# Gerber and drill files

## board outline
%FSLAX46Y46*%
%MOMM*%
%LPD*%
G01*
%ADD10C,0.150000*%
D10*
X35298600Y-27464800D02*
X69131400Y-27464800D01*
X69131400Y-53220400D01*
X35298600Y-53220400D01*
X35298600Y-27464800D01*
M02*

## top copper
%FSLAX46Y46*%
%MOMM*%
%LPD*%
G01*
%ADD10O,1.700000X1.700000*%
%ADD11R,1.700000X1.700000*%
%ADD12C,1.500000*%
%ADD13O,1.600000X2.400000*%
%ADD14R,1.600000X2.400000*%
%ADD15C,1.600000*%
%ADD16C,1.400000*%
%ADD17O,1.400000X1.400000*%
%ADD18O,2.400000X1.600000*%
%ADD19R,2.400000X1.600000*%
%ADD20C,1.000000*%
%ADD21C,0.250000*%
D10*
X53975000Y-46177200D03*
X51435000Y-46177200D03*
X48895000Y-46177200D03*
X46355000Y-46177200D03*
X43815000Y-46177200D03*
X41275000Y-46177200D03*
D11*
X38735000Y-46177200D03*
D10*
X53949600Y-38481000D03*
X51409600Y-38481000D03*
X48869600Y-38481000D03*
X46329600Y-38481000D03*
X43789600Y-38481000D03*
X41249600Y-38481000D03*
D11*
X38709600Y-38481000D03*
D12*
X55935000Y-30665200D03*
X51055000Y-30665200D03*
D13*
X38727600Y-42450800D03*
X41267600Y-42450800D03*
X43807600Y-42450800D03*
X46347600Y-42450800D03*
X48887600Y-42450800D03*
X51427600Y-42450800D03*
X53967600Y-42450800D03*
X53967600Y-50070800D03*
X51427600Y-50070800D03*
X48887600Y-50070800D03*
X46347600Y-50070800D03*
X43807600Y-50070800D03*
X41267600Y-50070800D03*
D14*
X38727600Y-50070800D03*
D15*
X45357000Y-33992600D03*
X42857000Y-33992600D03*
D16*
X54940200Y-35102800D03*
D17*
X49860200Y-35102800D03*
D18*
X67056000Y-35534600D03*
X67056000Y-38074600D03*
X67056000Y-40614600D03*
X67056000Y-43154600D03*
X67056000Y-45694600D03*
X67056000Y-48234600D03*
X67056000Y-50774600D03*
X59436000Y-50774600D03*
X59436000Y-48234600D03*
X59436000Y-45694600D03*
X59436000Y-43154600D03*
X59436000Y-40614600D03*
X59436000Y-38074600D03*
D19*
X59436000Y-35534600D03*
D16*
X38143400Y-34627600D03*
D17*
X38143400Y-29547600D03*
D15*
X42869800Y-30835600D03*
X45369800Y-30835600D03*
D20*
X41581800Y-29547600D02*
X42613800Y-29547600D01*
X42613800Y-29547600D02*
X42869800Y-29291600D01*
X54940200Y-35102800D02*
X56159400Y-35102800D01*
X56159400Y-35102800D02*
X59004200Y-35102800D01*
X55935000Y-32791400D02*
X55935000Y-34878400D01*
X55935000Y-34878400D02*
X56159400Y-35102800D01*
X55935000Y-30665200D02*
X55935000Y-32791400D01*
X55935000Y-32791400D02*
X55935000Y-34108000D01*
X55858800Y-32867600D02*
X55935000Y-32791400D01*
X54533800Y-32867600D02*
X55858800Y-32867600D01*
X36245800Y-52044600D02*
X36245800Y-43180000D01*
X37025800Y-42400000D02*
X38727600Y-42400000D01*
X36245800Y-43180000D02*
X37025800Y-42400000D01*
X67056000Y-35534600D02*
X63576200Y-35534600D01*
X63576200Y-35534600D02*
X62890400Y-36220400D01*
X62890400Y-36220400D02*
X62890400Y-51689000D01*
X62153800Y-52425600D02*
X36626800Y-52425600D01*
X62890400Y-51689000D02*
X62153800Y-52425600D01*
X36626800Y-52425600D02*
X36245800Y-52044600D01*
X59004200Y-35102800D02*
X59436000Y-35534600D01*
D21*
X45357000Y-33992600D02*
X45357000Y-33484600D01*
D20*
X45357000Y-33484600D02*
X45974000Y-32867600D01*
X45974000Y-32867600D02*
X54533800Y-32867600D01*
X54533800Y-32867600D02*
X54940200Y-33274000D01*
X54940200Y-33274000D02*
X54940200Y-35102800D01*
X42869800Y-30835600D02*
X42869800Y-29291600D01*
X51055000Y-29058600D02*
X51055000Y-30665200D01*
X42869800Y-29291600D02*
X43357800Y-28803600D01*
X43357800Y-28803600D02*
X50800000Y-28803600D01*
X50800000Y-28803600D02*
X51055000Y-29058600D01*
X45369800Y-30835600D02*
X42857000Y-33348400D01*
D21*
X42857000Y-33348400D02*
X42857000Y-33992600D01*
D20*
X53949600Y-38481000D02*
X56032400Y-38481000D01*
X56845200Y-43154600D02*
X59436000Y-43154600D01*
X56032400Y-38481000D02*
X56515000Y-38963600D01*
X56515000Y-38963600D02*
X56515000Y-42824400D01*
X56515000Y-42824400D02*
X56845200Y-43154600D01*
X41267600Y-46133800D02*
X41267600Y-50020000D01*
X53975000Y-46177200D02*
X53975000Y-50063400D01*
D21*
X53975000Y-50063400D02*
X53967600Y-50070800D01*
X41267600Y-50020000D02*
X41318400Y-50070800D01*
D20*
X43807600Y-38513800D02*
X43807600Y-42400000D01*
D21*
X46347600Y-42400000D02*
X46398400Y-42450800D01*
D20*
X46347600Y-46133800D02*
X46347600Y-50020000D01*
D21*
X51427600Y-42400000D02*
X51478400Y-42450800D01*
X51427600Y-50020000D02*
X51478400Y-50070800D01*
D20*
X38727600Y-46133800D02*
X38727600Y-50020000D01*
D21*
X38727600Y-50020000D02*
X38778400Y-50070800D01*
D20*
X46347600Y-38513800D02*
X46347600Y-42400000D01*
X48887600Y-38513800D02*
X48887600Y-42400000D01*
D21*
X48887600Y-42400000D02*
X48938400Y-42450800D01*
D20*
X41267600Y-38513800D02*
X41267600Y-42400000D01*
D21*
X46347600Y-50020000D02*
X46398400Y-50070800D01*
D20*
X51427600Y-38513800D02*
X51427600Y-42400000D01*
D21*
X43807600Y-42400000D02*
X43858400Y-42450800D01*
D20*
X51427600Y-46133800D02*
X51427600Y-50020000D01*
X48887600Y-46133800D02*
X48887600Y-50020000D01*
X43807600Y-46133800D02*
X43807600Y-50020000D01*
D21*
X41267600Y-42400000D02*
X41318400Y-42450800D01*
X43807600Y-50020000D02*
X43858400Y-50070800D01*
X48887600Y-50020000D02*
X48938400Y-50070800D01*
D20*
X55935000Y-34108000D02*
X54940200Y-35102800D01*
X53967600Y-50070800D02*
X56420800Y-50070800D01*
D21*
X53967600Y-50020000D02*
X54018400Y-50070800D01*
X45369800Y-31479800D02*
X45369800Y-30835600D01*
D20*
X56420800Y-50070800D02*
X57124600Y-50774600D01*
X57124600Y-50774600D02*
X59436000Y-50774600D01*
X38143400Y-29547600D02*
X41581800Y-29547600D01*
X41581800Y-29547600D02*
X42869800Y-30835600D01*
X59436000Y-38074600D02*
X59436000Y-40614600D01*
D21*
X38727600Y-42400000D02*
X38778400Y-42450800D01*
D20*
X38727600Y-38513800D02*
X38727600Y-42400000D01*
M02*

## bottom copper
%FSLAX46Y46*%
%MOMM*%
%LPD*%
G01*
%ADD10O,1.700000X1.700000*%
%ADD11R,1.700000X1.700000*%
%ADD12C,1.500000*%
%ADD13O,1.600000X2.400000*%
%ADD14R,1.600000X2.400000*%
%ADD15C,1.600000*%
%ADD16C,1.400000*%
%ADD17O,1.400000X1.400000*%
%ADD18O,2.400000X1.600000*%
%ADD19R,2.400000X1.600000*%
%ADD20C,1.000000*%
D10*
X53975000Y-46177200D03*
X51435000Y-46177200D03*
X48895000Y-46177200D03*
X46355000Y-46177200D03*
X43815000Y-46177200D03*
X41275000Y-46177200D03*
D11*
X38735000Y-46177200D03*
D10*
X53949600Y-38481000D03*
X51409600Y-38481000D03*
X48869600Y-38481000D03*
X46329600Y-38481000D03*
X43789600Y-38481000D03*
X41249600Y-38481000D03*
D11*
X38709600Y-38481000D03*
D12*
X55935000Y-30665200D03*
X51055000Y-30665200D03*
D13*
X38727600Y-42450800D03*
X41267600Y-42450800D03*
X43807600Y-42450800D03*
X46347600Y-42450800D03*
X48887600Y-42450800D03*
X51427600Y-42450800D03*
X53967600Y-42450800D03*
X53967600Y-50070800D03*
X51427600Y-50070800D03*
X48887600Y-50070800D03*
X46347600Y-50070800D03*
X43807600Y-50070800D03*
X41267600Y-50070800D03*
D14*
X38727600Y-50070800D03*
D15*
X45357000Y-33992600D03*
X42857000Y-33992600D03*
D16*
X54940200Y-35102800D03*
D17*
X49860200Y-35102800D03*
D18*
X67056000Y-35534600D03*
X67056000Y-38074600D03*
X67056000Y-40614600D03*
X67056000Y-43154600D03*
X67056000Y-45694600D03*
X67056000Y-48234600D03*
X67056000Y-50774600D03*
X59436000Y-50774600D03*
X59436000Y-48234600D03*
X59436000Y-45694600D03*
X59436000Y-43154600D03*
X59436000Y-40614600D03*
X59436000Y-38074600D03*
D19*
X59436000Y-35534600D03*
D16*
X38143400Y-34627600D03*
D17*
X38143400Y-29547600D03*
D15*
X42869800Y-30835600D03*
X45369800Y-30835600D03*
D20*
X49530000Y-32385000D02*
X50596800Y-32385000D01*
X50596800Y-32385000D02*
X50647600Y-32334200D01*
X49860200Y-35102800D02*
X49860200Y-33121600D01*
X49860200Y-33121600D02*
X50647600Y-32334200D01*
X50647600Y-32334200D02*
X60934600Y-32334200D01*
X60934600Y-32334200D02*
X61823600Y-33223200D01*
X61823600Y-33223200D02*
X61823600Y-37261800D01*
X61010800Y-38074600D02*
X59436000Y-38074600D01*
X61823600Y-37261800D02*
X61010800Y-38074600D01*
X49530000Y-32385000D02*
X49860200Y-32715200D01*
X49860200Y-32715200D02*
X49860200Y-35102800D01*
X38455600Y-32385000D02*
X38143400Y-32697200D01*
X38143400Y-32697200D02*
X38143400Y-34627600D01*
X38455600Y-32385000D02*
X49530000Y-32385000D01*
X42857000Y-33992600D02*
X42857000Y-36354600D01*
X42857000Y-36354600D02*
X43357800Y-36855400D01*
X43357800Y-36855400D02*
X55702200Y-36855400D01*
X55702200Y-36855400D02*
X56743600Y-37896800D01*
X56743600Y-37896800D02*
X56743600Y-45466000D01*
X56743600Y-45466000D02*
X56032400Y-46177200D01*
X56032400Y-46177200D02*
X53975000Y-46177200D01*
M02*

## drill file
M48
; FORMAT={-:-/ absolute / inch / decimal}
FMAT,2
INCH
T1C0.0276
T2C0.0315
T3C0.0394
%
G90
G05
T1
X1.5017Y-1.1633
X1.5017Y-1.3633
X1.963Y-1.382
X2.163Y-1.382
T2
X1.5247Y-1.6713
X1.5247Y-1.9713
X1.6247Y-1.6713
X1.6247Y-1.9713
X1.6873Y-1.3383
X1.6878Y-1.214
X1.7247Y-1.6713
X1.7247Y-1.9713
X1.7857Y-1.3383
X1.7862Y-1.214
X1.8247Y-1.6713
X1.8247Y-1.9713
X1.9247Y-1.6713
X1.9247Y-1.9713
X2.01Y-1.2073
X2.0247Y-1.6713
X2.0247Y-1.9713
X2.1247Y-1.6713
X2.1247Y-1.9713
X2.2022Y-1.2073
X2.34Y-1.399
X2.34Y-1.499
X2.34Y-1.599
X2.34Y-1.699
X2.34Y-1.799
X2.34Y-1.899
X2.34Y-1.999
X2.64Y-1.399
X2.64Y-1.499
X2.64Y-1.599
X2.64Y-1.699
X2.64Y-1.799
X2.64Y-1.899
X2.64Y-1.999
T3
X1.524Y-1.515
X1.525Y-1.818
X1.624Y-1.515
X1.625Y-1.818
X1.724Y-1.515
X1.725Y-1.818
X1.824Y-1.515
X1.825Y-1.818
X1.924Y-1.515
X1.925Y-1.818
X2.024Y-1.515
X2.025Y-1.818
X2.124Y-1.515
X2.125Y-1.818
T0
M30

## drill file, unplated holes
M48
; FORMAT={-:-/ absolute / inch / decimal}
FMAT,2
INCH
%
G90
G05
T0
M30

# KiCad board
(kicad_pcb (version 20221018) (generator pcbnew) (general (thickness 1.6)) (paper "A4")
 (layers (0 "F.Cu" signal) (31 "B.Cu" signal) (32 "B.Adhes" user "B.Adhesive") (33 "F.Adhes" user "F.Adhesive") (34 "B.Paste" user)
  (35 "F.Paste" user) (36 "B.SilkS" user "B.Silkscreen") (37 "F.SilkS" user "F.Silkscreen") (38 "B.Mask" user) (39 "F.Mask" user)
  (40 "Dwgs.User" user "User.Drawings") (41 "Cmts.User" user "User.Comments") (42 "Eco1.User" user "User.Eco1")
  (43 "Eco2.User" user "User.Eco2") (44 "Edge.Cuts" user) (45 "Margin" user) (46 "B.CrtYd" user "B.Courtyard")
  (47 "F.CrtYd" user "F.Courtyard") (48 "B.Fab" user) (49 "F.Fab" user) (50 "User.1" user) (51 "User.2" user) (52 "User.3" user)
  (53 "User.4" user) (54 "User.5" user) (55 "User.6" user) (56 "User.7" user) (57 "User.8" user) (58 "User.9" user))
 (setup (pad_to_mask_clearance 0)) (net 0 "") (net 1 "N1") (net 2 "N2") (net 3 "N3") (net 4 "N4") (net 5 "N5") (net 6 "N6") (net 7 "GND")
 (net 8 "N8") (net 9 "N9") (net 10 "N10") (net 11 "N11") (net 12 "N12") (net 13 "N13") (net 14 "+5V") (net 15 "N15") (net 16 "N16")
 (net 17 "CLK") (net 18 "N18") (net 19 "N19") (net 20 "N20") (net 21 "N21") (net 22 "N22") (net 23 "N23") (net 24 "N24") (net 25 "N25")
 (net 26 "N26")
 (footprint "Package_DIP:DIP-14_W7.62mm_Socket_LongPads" (layer "F.Cu") (at 38.7276 50.0708 90)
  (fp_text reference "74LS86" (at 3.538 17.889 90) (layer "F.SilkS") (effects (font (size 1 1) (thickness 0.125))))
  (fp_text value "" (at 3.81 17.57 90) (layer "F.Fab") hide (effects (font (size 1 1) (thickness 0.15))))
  (pad "1" thru_hole rect (at 0 0 90) (size 2.4 1.6) (drill 0.8) (layers "*.Cu" "*.Mask") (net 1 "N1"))
  (pad "2" thru_hole oval (at 0 2.54 90) (size 2.4 1.6) (drill 0.8) (layers "*.Cu" "*.Mask") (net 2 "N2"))
  (pad "3" thru_hole oval (at 0 5.08 90) (size 2.4 1.6) (drill 0.8) (layers "*.Cu" "*.Mask") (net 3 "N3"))
  (pad "4" thru_hole oval (at 0 7.62 90) (size 2.4 1.6) (drill 0.8) (layers "*.Cu" "*.Mask") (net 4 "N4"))
  (pad "5" thru_hole oval (at 0 10.16 90) (size 2.4 1.6) (drill 0.8) (layers "*.Cu" "*.Mask") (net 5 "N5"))
  (pad "6" thru_hole oval (at 0 12.7 90) (size 2.4 1.6) (drill 0.8) (layers "*.Cu" "*.Mask") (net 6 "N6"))
  (pad "7" thru_hole oval (at 0 15.24 90) (size 2.4 1.6) (drill 0.8) (layers "*.Cu" "*.Mask") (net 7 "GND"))
  (pad "8" thru_hole oval (at 7.62 15.24 90) (size 2.4 1.6) (drill 0.8) (layers "*.Cu" "*.Mask") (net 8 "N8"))
  (pad "9" thru_hole oval (at 7.62 12.7 90) (size 2.4 1.6) (drill 0.8) (layers "*.Cu" "*.Mask") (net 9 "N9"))
  (pad "10" thru_hole oval (at 7.62 10.16 90) (size 2.4 1.6) (drill 0.8) (layers "*.Cu" "*.Mask") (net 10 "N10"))
  (pad "11" thru_hole oval (at 7.62 7.62 90) (size 2.4 1.6) (drill 0.8) (layers "*.Cu" "*.Mask") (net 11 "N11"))
  (pad "12" thru_hole oval (at 7.62 5.08 90) (size 2.4 1.6) (drill 0.8) (layers "*.Cu" "*.Mask") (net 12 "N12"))
  (pad "13" thru_hole oval (at 7.62 2.54 90) (size 2.4 1.6) (drill 0.8) (layers "*.Cu" "*.Mask") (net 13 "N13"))
  (pad "14" thru_hole oval (at 7.62 0 90) (size 2.4 1.6) (drill 0.8) (layers "*.Cu" "*.Mask") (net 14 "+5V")))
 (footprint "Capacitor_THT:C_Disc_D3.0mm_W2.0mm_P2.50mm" (layer "F.Cu") (at 45.357 33.9926 180)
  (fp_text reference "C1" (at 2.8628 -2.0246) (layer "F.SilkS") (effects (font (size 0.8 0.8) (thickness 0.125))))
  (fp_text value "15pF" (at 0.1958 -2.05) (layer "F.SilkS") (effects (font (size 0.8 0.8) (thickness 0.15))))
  (pad "1" thru_hole circle (at 0 0 180) (size 1.6 1.6) (drill 0.8) (layers "*.Cu" "*.Mask") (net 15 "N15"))
  (pad "2" thru_hole circle (at 2.5 0 180) (size 1.6 1.6) (drill 0.8) (layers "*.Cu" "*.Mask") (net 7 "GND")))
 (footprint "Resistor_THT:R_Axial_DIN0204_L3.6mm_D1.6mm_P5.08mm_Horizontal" (layer "F.Cu") (at 54.9402 35.1028 180)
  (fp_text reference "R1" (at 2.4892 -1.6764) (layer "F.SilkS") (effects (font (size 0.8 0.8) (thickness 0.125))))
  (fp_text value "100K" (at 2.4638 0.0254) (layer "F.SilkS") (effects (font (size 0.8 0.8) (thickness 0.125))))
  (pad "1" thru_hole circle (at 0 0 180) (size 1.4 1.4) (drill 0.7) (layers "*.Cu" "*.Mask") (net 15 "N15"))
  (pad "2" thru_hole oval (at 5.08 0 180) (size 1.4 1.4) (drill 0.7) (layers "*.Cu" "*.Mask") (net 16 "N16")))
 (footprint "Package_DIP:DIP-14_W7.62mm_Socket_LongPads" (layer "F.Cu") (at 59.436 35.5346)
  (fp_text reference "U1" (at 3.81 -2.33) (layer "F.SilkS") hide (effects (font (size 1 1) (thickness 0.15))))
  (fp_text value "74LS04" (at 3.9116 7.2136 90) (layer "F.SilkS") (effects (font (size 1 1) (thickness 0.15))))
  (pad "1" thru_hole rect (at 0 0) (size 2.4 1.6) (drill 0.8) (layers "*.Cu" "*.Mask") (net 15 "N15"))
  (pad "2" thru_hole oval (at 0 2.54) (size 2.4 1.6) (drill 0.8) (layers "*.Cu" "*.Mask") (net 16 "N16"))
  (pad "3" thru_hole oval (at 0 5.08) (size 2.4 1.6) (drill 0.8) (layers "*.Cu" "*.Mask") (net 16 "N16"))
  (pad "4" thru_hole oval (at 0 7.62) (size 2.4 1.6) (drill 0.8) (layers "*.Cu" "*.Mask") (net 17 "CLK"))
  (pad "5" thru_hole oval (at 0 10.16) (size 2.4 1.6) (drill 0.8) (layers "*.Cu" "*.Mask") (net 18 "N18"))
  (pad "6" thru_hole oval (at 0 12.7) (size 2.4 1.6) (drill 0.8) (layers "*.Cu" "*.Mask") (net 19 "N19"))
  (pad "7" thru_hole oval (at 0 15.24) (size 2.4 1.6) (drill 0.8) (layers "*.Cu" "*.Mask") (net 7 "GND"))
  (pad "8" thru_hole oval (at 7.62 15.24) (size 2.4 1.6) (drill 0.8) (layers "*.Cu" "*.Mask") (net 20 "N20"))
  (pad "9" thru_hole oval (at 7.62 12.7) (size 2.4 1.6) (drill 0.8) (layers "*.Cu" "*.Mask") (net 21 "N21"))
  (pad "10" thru_hole oval (at 7.62 10.16) (size 2.4 1.6) (drill 0.8) (layers "*.Cu" "*.Mask") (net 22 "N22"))
  (pad "11" thru_hole oval (at 7.62 7.62) (size 2.4 1.6) (drill 0.8) (layers "*.Cu" "*.Mask") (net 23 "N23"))
  (pad "12" thru_hole oval (at 7.62 5.08) (size 2.4 1.6) (drill 0.8) (layers "*.Cu" "*.Mask") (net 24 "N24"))
  (pad "13" thru_hole oval (at 7.62 2.54) (size 2.4 1.6) (drill 0.8) (layers "*.Cu" "*.Mask") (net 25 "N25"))
  (pad "14" thru_hole oval (at 7.62 0) (size 2.4 1.6) (drill 0.8) (layers "*.Cu" "*.Mask") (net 14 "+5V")))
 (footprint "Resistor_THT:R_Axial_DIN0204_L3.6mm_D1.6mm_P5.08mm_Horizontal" (layer "F.Cu") (at 38.1434 34.6276 90)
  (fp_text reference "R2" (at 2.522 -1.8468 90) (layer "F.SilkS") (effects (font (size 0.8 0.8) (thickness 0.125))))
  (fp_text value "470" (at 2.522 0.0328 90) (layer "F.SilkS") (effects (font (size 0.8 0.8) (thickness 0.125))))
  (pad "1" thru_hole circle (at 0 0 90) (size 1.4 1.4) (drill 0.7) (layers "*.Cu" "*.Mask") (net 16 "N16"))
  (pad "2" thru_hole oval (at 5.08 0 90) (size 1.4 1.4) (drill 0.7) (layers "*.Cu" "*.Mask") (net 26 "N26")))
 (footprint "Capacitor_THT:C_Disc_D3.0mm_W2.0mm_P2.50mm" (layer "F.Cu") (at 42.8698 30.8356)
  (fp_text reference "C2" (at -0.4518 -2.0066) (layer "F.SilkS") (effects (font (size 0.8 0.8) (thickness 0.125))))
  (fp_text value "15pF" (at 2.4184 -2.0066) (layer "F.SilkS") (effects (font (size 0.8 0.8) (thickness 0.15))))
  (pad "1" thru_hole circle (at 0 0) (size 1.6 1.6) (drill 0.8) (layers "*.Cu" "*.Mask") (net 26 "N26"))
  (pad "2" thru_hole circle (at 2.5 0) (size 1.6 1.6) (drill 0.8) (layers "*.Cu" "*.Mask") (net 7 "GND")))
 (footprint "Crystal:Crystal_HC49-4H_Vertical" (layer "F.Cu") (at 55.935 30.6652 180)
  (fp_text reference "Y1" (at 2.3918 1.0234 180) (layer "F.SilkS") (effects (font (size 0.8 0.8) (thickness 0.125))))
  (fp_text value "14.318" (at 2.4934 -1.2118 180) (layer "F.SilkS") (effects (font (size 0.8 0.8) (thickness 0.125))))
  (pad "1" thru_hole circle (at 0 0 180) (size 1.5 1.5) (drill 0.8) (layers "*.Cu" "*.Mask") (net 15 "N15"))
  (pad "2" thru_hole circle (at 4.88 0 180) (size 1.5 1.5) (drill 0.8) (layers "*.Cu" "*.Mask") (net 26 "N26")))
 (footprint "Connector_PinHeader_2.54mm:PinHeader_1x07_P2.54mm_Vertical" (layer "B.Cu") (at 38.735 46.1772 -90)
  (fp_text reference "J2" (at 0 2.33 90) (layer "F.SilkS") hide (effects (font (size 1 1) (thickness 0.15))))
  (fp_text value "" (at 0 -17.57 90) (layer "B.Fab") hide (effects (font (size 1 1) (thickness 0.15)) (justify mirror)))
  (pad "1" thru_hole rect (at 0 0 270) (size 1.7 1.7) (drill 1) (layers "*.Cu" "*.Mask") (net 1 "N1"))
  (pad "2" thru_hole oval (at 0 -2.54 270) (size 1.7 1.7) (drill 1) (layers "*.Cu" "*.Mask") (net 2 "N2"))
  (pad "3" thru_hole oval (at 0 -5.08 270) (size 1.7 1.7) (drill 1) (layers "*.Cu" "*.Mask") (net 3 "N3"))
  (pad "4" thru_hole oval (at 0 -7.62 270) (size 1.7 1.7) (drill 1) (layers "*.Cu" "*.Mask") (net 4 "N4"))
  (pad "5" thru_hole oval (at 0 -10.16 270) (size 1.7 1.7) (drill 1) (layers "*.Cu" "*.Mask") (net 5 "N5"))
  (pad "6" thru_hole oval (at 0 -12.7 270) (size 1.7 1.7) (drill 1) (layers "*.Cu" "*.Mask") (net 6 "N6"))
  (pad "7" thru_hole oval (at 0 -15.24 270) (size 1.7 1.7) (drill 1) (layers "*.Cu" "*.Mask") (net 7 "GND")))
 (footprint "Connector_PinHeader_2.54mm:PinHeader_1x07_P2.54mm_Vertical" (layer "B.Cu") (at 38.7096 38.481 -90)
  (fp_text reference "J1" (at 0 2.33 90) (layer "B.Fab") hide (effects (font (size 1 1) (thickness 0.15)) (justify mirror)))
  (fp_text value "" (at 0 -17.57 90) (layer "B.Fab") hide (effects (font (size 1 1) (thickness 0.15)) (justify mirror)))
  (pad "1" thru_hole rect (at 0 0 270) (size 1.7 1.7) (drill 1) (layers "*.Cu" "*.Mask") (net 14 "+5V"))
  (pad "2" thru_hole oval (at 0 -2.54 270) (size 1.7 1.7) (drill 1) (layers "*.Cu" "*.Mask") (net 13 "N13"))
  (pad "3" thru_hole oval (at 0 -5.08 270) (size 1.7 1.7) (drill 1) (layers "*.Cu" "*.Mask") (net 12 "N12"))
  (pad "4" thru_hole oval (at 0 -7.62 270) (size 1.7 1.7) (drill 1) (layers "*.Cu" "*.Mask") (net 11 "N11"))
  (pad "5" thru_hole oval (at 0 -10.16 270) (size 1.7 1.7) (drill 1) (layers "*.Cu" "*.Mask") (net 10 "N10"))
  (pad "6" thru_hole oval (at 0 -12.7 270) (size 1.7 1.7) (drill 1) (layers "*.Cu" "*.Mask") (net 9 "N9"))
  (pad "7" thru_hole oval (at 0 -15.24 270) (size 1.7 1.7) (drill 1) (layers "*.Cu" "*.Mask") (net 17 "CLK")))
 (gr_rect (start 35.2986 27.4648) (end 69.1314 53.2204) (stroke (width 0.15) (type default)) (fill none) (layer "Edge.Cuts"))
 (segment (start 55.935 32.7914) (end 55.935 34.8784) (width 1) (layer "F.Cu") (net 15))
 (segment (start 54.5338 32.8676) (end 55.8588 32.8676) (width 1) (layer "F.Cu") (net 15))
 (segment (start 56.1594 35.1028) (end 59.0042 35.1028) (width 1) (layer "F.Cu") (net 15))
 (segment (start 45.974 32.8676) (end 54.5338 32.8676) (width 1) (layer "F.Cu") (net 15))
 (segment (start 55.935 34.108) (end 54.9402 35.1028) (width 1) (layer "F.Cu") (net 15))
 (segment (start 55.935 32.7914) (end 55.935 34.108) (width 1) (layer "F.Cu") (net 15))
 (segment (start 55.935 34.8784) (end 56.1594 35.1028) (width 1) (layer "F.Cu") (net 15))
 (segment (start 45.357 33.9926) (end 45.357 33.4846) (width 0.25) (layer "F.Cu") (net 15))
 (segment (start 55.935 30.6652) (end 55.935 32.7914) (width 1) (layer "F.Cu") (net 15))
 (segment (start 55.8588 32.8676) (end 55.935 32.7914) (width 1) (layer "F.Cu") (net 15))
 (segment (start 54.5338 32.8676) (end 54.9402 33.274) (width 1) (layer "F.Cu") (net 15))
 (segment (start 54.9402 35.1028) (end 56.1594 35.1028) (width 1) (layer "F.Cu") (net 15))
 (segment (start 45.357 33.4846) (end 45.974 32.8676) (width 1) (layer "F.Cu") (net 15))
 (segment (start 59.0042 35.1028) (end 59.436 35.5346) (width 1) (layer "F.Cu") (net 15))
 (segment (start 54.9402 33.274) (end 54.9402 35.1028) (width 1) (layer "F.Cu") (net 15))
 (segment (start 53.9676 50.0708) (end 56.4208 50.0708) (width 1) (layer "F.Cu") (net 7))
 (segment (start 53.9676 50.02) (end 54.0184 50.0708) (width 0.25) (layer "F.Cu") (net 7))
 (segment (start 45.3698 30.8356) (end 42.857 33.3484) (width 1) (layer "F.Cu") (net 7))
 (segment (start 45.3698 31.4798) (end 45.3698 30.8356) (width 0.25) (layer "F.Cu") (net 7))
 (segment (start 53.975 50.0634) (end 53.9676 50.0708) (width 0.25) (layer "F.Cu") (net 7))
 (segment (start 56.4208 50.0708) (end 57.1246 50.7746) (width 1) (layer "F.Cu") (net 7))
 (segment (start 53.975 46.1772) (end 53.975 50.0634) (width 1) (layer "F.Cu") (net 7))
 (segment (start 42.857 33.3484) (end 42.857 33.9926) (width 0.25) (layer "F.Cu") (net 7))
 (segment (start 57.1246 50.7746) (end 59.436 50.7746) (width 1) (layer "F.Cu") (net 7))
 (segment (start 42.857 36.3546) (end 43.3578 36.8554) (width 1) (layer "B.Cu") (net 7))
 (segment (start 55.7022 36.8554) (end 56.7436 37.8968) (width 1) (layer "B.Cu") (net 7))
 (segment (start 42.857 33.9926) (end 42.857 36.3546) (width 1) (layer "B.Cu") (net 7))
 (segment (start 56.7436 45.466) (end 56.0324 46.1772) (width 1) (layer "B.Cu") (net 7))
 (segment (start 56.7436 37.8968) (end 56.7436 45.466) (width 1) (layer "B.Cu") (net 7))
 (segment (start 56.0324 46.1772) (end 53.975 46.1772) (width 1) (layer "B.Cu") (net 7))
 (segment (start 43.3578 36.8554) (end 55.7022 36.8554) (width 1) (layer "B.Cu") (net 7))
 (segment (start 38.1434 29.5476) (end 41.5818 29.5476) (width 1) (layer "F.Cu") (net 26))
 (segment (start 42.6138 29.5476) (end 42.8698 29.2916) (width 1) (layer "F.Cu") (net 26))
 (segment (start 51.055 29.0586) (end 51.055 30.6652) (width 1) (layer "F.Cu") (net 26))
 (segment (start 41.5818 29.5476) (end 42.6138 29.5476) (width 1) (layer "F.Cu") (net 26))
 (segment (start 42.8698 29.2916) (end 43.3578 28.8036) (width 1) (layer "F.Cu") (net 26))
 (segment (start 43.3578 28.8036) (end 50.8 28.8036) (width 1) (layer "F.Cu") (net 26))
 (segment (start 50.8 28.8036) (end 51.055 29.0586) (width 1) (layer "F.Cu") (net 26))
 (segment (start 41.5818 29.5476) (end 42.8698 30.8356) (width 1) (layer "F.Cu") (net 26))
 (segment (start 42.8698 30.8356) (end 42.8698 29.2916) (width 1) (layer "F.Cu") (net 26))
 (segment (start 59.436 38.0746) (end 59.436 40.6146) (width 1) (layer "F.Cu") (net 16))
 (segment (start 50.6476 32.3342) (end 60.9346 32.3342) (width 1) (layer "B.Cu") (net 16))
 (segment (start 49.8602 35.1028) (end 49.8602 33.1216) (width 1) (layer "B.Cu") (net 16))
 (segment (start 61.8236 37.2618) (end 61.0108 38.0746) (width 1) (layer "B.Cu") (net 16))
 (segment (start 60.9346 32.3342) (end 61.8236 33.2232) (width 1) (layer "B.Cu") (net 16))
 (segment (start 49.8602 32.7152) (end 49.8602 35.1028) (width 1) (layer "B.Cu") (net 16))
 (segment (start 61.0108 38.0746) (end 59.436 38.0746) (width 1) (layer "B.Cu") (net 16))
 (segment (start 61.8236 33.2232) (end 61.8236 37.2618) (width 1) (layer "B.Cu") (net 16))
 (segment (start 38.4556 32.385) (end 49.53 32.385) (width 1) (layer "B.Cu") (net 16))
 (segment (start 38.1434 32.6972) (end 38.1434 34.6276) (width 1) (layer "B.Cu") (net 16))
 (segment (start 49.53 32.385) (end 50.5968 32.385) (width 1) (layer "B.Cu") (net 16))
 (segment (start 49.53 32.385) (end 49.8602 32.7152) (width 1) (layer "B.Cu") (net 16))
 (segment (start 38.4556 32.385) (end 38.1434 32.6972) (width 1) (layer "B.Cu") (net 16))
 (segment (start 49.8602 33.1216) (end 50.6476 32.3342) (width 1) (layer "B.Cu") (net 16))
 (segment (start 50.5968 32.385) (end 50.6476 32.3342) (width 1) (layer "B.Cu") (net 16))
 (segment (start 62.1538 52.4256) (end 36.6268 52.4256) (width 1) (layer "F.Cu") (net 14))
 (segment (start 37.0258 42.4) (end 38.7276 42.4) (width 1) (layer "F.Cu") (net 14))
 (segment (start 36.2458 52.0446) (end 36.2458 43.18) (width 1) (layer "F.Cu") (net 14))
 (segment (start 36.2458 43.18) (end 37.0258 42.4) (width 1) (layer "F.Cu") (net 14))
 (segment (start 38.7276 42.4) (end 38.7784 42.4508) (width 0.25) (layer "F.Cu") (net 14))
 (segment (start 67.056 35.5346) (end 63.5762 35.5346) (width 1) (layer "F.Cu") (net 14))
 (segment (start 36.6268 52.4256) (end 36.2458 52.0446) (width 1) (layer "F.Cu") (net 14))
 (segment (start 62.8904 36.2204) (end 62.8904 51.689) (width 1) (layer "F.Cu") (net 14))
 (segment (start 62.8904 51.689) (end 62.1538 52.4256) (width 1) (layer "F.Cu") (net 14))
 (segment (start 63.5762 35.5346) (end 62.8904 36.2204) (width 1) (layer "F.Cu") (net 14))
 (segment (start 38.7276 38.5138) (end 38.7276 42.4) (width 1) (layer "F.Cu") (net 14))
 (segment (start 56.8452 43.1546) (end 59.436 43.1546) (width 1) (layer "F.Cu") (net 17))
 (segment (start 56.515 38.9636) (end 56.515 42.8244) (width 1) (layer "F.Cu") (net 17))
 (segment (start 53.9496 38.481) (end 56.0324 38.481) (width 1) (layer "F.Cu") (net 17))
 (segment (start 56.515 42.8244) (end 56.8452 43.1546) (width 1) (layer "F.Cu") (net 17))
 (segment (start 56.0324 38.481) (end 56.515 38.9636) (width 1) (layer "F.Cu") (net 17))
 (segment (start 38.7276 46.1338) (end 38.7276 50.02) (width 1) (layer "F.Cu") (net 1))
 (segment (start 38.7276 50.02) (end 38.7784 50.0708) (width 0.25) (layer "F.Cu") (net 1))
 (segment (start 41.2676 50.02) (end 41.3184 50.0708) (width 0.25) (layer "F.Cu") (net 2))
 (segment (start 41.2676 46.1338) (end 41.2676 50.02) (width 1) (layer "F.Cu") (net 2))
 (segment (start 43.8076 46.1338) (end 43.8076 50.02) (width 1) (layer "F.Cu") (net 3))
 (segment (start 43.8076 50.02) (end 43.8584 50.0708) (width 0.25) (layer "F.Cu") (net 3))
 (segment (start 46.3476 46.1338) (end 46.3476 50.02) (width 1) (layer "F.Cu") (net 4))
 (segment (start 46.3476 50.02) (end 46.3984 50.0708) (width 0.25) (layer "F.Cu") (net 4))
 (segment (start 48.8876 46.1338) (end 48.8876 50.02) (width 1) (layer "F.Cu") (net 5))
 (segment (start 48.8876 50.02) (end 48.9384 50.0708) (width 0.25) (layer "F.Cu") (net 5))
 (segment (start 51.4276 50.02) (end 51.4784 50.0708) (width 0.25) (layer "F.Cu") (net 6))
 (segment (start 51.4276 46.1338) (end 51.4276 50.02) (width 1) (layer "F.Cu") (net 6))
 (segment (start 51.4276 42.4) (end 51.4784 42.4508) (width 0.25) (layer "F.Cu") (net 9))
 (segment (start 51.4276 38.5138) (end 51.4276 42.4) (width 1) (layer "F.Cu") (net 9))
 (segment (start 48.8876 38.5138) (end 48.8876 42.4) (width 1) (layer "F.Cu") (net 10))
 (segment (start 48.8876 42.4) (end 48.9384 42.4508) (width 0.25) (layer "F.Cu") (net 10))
 (segment (start 46.3476 42.4) (end 46.3984 42.4508) (width 0.25) (layer "F.Cu") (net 11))
 (segment (start 46.3476 38.5138) (end 46.3476 42.4) (width 1) (layer "F.Cu") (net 11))
 (segment (start 43.8076 38.5138) (end 43.8076 42.4) (width 1) (layer "F.Cu") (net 12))
 (segment (start 43.8076 42.4) (end 43.8584 42.4508) (width 0.25) (layer "F.Cu") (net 12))
 (segment (start 41.2676 38.5138) (end 41.2676 42.4) (width 1) (layer "F.Cu") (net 13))
 (segment (start 41.2676 42.4) (end 41.3184 42.4508) (width 0.25) (layer "F.Cu") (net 13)))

